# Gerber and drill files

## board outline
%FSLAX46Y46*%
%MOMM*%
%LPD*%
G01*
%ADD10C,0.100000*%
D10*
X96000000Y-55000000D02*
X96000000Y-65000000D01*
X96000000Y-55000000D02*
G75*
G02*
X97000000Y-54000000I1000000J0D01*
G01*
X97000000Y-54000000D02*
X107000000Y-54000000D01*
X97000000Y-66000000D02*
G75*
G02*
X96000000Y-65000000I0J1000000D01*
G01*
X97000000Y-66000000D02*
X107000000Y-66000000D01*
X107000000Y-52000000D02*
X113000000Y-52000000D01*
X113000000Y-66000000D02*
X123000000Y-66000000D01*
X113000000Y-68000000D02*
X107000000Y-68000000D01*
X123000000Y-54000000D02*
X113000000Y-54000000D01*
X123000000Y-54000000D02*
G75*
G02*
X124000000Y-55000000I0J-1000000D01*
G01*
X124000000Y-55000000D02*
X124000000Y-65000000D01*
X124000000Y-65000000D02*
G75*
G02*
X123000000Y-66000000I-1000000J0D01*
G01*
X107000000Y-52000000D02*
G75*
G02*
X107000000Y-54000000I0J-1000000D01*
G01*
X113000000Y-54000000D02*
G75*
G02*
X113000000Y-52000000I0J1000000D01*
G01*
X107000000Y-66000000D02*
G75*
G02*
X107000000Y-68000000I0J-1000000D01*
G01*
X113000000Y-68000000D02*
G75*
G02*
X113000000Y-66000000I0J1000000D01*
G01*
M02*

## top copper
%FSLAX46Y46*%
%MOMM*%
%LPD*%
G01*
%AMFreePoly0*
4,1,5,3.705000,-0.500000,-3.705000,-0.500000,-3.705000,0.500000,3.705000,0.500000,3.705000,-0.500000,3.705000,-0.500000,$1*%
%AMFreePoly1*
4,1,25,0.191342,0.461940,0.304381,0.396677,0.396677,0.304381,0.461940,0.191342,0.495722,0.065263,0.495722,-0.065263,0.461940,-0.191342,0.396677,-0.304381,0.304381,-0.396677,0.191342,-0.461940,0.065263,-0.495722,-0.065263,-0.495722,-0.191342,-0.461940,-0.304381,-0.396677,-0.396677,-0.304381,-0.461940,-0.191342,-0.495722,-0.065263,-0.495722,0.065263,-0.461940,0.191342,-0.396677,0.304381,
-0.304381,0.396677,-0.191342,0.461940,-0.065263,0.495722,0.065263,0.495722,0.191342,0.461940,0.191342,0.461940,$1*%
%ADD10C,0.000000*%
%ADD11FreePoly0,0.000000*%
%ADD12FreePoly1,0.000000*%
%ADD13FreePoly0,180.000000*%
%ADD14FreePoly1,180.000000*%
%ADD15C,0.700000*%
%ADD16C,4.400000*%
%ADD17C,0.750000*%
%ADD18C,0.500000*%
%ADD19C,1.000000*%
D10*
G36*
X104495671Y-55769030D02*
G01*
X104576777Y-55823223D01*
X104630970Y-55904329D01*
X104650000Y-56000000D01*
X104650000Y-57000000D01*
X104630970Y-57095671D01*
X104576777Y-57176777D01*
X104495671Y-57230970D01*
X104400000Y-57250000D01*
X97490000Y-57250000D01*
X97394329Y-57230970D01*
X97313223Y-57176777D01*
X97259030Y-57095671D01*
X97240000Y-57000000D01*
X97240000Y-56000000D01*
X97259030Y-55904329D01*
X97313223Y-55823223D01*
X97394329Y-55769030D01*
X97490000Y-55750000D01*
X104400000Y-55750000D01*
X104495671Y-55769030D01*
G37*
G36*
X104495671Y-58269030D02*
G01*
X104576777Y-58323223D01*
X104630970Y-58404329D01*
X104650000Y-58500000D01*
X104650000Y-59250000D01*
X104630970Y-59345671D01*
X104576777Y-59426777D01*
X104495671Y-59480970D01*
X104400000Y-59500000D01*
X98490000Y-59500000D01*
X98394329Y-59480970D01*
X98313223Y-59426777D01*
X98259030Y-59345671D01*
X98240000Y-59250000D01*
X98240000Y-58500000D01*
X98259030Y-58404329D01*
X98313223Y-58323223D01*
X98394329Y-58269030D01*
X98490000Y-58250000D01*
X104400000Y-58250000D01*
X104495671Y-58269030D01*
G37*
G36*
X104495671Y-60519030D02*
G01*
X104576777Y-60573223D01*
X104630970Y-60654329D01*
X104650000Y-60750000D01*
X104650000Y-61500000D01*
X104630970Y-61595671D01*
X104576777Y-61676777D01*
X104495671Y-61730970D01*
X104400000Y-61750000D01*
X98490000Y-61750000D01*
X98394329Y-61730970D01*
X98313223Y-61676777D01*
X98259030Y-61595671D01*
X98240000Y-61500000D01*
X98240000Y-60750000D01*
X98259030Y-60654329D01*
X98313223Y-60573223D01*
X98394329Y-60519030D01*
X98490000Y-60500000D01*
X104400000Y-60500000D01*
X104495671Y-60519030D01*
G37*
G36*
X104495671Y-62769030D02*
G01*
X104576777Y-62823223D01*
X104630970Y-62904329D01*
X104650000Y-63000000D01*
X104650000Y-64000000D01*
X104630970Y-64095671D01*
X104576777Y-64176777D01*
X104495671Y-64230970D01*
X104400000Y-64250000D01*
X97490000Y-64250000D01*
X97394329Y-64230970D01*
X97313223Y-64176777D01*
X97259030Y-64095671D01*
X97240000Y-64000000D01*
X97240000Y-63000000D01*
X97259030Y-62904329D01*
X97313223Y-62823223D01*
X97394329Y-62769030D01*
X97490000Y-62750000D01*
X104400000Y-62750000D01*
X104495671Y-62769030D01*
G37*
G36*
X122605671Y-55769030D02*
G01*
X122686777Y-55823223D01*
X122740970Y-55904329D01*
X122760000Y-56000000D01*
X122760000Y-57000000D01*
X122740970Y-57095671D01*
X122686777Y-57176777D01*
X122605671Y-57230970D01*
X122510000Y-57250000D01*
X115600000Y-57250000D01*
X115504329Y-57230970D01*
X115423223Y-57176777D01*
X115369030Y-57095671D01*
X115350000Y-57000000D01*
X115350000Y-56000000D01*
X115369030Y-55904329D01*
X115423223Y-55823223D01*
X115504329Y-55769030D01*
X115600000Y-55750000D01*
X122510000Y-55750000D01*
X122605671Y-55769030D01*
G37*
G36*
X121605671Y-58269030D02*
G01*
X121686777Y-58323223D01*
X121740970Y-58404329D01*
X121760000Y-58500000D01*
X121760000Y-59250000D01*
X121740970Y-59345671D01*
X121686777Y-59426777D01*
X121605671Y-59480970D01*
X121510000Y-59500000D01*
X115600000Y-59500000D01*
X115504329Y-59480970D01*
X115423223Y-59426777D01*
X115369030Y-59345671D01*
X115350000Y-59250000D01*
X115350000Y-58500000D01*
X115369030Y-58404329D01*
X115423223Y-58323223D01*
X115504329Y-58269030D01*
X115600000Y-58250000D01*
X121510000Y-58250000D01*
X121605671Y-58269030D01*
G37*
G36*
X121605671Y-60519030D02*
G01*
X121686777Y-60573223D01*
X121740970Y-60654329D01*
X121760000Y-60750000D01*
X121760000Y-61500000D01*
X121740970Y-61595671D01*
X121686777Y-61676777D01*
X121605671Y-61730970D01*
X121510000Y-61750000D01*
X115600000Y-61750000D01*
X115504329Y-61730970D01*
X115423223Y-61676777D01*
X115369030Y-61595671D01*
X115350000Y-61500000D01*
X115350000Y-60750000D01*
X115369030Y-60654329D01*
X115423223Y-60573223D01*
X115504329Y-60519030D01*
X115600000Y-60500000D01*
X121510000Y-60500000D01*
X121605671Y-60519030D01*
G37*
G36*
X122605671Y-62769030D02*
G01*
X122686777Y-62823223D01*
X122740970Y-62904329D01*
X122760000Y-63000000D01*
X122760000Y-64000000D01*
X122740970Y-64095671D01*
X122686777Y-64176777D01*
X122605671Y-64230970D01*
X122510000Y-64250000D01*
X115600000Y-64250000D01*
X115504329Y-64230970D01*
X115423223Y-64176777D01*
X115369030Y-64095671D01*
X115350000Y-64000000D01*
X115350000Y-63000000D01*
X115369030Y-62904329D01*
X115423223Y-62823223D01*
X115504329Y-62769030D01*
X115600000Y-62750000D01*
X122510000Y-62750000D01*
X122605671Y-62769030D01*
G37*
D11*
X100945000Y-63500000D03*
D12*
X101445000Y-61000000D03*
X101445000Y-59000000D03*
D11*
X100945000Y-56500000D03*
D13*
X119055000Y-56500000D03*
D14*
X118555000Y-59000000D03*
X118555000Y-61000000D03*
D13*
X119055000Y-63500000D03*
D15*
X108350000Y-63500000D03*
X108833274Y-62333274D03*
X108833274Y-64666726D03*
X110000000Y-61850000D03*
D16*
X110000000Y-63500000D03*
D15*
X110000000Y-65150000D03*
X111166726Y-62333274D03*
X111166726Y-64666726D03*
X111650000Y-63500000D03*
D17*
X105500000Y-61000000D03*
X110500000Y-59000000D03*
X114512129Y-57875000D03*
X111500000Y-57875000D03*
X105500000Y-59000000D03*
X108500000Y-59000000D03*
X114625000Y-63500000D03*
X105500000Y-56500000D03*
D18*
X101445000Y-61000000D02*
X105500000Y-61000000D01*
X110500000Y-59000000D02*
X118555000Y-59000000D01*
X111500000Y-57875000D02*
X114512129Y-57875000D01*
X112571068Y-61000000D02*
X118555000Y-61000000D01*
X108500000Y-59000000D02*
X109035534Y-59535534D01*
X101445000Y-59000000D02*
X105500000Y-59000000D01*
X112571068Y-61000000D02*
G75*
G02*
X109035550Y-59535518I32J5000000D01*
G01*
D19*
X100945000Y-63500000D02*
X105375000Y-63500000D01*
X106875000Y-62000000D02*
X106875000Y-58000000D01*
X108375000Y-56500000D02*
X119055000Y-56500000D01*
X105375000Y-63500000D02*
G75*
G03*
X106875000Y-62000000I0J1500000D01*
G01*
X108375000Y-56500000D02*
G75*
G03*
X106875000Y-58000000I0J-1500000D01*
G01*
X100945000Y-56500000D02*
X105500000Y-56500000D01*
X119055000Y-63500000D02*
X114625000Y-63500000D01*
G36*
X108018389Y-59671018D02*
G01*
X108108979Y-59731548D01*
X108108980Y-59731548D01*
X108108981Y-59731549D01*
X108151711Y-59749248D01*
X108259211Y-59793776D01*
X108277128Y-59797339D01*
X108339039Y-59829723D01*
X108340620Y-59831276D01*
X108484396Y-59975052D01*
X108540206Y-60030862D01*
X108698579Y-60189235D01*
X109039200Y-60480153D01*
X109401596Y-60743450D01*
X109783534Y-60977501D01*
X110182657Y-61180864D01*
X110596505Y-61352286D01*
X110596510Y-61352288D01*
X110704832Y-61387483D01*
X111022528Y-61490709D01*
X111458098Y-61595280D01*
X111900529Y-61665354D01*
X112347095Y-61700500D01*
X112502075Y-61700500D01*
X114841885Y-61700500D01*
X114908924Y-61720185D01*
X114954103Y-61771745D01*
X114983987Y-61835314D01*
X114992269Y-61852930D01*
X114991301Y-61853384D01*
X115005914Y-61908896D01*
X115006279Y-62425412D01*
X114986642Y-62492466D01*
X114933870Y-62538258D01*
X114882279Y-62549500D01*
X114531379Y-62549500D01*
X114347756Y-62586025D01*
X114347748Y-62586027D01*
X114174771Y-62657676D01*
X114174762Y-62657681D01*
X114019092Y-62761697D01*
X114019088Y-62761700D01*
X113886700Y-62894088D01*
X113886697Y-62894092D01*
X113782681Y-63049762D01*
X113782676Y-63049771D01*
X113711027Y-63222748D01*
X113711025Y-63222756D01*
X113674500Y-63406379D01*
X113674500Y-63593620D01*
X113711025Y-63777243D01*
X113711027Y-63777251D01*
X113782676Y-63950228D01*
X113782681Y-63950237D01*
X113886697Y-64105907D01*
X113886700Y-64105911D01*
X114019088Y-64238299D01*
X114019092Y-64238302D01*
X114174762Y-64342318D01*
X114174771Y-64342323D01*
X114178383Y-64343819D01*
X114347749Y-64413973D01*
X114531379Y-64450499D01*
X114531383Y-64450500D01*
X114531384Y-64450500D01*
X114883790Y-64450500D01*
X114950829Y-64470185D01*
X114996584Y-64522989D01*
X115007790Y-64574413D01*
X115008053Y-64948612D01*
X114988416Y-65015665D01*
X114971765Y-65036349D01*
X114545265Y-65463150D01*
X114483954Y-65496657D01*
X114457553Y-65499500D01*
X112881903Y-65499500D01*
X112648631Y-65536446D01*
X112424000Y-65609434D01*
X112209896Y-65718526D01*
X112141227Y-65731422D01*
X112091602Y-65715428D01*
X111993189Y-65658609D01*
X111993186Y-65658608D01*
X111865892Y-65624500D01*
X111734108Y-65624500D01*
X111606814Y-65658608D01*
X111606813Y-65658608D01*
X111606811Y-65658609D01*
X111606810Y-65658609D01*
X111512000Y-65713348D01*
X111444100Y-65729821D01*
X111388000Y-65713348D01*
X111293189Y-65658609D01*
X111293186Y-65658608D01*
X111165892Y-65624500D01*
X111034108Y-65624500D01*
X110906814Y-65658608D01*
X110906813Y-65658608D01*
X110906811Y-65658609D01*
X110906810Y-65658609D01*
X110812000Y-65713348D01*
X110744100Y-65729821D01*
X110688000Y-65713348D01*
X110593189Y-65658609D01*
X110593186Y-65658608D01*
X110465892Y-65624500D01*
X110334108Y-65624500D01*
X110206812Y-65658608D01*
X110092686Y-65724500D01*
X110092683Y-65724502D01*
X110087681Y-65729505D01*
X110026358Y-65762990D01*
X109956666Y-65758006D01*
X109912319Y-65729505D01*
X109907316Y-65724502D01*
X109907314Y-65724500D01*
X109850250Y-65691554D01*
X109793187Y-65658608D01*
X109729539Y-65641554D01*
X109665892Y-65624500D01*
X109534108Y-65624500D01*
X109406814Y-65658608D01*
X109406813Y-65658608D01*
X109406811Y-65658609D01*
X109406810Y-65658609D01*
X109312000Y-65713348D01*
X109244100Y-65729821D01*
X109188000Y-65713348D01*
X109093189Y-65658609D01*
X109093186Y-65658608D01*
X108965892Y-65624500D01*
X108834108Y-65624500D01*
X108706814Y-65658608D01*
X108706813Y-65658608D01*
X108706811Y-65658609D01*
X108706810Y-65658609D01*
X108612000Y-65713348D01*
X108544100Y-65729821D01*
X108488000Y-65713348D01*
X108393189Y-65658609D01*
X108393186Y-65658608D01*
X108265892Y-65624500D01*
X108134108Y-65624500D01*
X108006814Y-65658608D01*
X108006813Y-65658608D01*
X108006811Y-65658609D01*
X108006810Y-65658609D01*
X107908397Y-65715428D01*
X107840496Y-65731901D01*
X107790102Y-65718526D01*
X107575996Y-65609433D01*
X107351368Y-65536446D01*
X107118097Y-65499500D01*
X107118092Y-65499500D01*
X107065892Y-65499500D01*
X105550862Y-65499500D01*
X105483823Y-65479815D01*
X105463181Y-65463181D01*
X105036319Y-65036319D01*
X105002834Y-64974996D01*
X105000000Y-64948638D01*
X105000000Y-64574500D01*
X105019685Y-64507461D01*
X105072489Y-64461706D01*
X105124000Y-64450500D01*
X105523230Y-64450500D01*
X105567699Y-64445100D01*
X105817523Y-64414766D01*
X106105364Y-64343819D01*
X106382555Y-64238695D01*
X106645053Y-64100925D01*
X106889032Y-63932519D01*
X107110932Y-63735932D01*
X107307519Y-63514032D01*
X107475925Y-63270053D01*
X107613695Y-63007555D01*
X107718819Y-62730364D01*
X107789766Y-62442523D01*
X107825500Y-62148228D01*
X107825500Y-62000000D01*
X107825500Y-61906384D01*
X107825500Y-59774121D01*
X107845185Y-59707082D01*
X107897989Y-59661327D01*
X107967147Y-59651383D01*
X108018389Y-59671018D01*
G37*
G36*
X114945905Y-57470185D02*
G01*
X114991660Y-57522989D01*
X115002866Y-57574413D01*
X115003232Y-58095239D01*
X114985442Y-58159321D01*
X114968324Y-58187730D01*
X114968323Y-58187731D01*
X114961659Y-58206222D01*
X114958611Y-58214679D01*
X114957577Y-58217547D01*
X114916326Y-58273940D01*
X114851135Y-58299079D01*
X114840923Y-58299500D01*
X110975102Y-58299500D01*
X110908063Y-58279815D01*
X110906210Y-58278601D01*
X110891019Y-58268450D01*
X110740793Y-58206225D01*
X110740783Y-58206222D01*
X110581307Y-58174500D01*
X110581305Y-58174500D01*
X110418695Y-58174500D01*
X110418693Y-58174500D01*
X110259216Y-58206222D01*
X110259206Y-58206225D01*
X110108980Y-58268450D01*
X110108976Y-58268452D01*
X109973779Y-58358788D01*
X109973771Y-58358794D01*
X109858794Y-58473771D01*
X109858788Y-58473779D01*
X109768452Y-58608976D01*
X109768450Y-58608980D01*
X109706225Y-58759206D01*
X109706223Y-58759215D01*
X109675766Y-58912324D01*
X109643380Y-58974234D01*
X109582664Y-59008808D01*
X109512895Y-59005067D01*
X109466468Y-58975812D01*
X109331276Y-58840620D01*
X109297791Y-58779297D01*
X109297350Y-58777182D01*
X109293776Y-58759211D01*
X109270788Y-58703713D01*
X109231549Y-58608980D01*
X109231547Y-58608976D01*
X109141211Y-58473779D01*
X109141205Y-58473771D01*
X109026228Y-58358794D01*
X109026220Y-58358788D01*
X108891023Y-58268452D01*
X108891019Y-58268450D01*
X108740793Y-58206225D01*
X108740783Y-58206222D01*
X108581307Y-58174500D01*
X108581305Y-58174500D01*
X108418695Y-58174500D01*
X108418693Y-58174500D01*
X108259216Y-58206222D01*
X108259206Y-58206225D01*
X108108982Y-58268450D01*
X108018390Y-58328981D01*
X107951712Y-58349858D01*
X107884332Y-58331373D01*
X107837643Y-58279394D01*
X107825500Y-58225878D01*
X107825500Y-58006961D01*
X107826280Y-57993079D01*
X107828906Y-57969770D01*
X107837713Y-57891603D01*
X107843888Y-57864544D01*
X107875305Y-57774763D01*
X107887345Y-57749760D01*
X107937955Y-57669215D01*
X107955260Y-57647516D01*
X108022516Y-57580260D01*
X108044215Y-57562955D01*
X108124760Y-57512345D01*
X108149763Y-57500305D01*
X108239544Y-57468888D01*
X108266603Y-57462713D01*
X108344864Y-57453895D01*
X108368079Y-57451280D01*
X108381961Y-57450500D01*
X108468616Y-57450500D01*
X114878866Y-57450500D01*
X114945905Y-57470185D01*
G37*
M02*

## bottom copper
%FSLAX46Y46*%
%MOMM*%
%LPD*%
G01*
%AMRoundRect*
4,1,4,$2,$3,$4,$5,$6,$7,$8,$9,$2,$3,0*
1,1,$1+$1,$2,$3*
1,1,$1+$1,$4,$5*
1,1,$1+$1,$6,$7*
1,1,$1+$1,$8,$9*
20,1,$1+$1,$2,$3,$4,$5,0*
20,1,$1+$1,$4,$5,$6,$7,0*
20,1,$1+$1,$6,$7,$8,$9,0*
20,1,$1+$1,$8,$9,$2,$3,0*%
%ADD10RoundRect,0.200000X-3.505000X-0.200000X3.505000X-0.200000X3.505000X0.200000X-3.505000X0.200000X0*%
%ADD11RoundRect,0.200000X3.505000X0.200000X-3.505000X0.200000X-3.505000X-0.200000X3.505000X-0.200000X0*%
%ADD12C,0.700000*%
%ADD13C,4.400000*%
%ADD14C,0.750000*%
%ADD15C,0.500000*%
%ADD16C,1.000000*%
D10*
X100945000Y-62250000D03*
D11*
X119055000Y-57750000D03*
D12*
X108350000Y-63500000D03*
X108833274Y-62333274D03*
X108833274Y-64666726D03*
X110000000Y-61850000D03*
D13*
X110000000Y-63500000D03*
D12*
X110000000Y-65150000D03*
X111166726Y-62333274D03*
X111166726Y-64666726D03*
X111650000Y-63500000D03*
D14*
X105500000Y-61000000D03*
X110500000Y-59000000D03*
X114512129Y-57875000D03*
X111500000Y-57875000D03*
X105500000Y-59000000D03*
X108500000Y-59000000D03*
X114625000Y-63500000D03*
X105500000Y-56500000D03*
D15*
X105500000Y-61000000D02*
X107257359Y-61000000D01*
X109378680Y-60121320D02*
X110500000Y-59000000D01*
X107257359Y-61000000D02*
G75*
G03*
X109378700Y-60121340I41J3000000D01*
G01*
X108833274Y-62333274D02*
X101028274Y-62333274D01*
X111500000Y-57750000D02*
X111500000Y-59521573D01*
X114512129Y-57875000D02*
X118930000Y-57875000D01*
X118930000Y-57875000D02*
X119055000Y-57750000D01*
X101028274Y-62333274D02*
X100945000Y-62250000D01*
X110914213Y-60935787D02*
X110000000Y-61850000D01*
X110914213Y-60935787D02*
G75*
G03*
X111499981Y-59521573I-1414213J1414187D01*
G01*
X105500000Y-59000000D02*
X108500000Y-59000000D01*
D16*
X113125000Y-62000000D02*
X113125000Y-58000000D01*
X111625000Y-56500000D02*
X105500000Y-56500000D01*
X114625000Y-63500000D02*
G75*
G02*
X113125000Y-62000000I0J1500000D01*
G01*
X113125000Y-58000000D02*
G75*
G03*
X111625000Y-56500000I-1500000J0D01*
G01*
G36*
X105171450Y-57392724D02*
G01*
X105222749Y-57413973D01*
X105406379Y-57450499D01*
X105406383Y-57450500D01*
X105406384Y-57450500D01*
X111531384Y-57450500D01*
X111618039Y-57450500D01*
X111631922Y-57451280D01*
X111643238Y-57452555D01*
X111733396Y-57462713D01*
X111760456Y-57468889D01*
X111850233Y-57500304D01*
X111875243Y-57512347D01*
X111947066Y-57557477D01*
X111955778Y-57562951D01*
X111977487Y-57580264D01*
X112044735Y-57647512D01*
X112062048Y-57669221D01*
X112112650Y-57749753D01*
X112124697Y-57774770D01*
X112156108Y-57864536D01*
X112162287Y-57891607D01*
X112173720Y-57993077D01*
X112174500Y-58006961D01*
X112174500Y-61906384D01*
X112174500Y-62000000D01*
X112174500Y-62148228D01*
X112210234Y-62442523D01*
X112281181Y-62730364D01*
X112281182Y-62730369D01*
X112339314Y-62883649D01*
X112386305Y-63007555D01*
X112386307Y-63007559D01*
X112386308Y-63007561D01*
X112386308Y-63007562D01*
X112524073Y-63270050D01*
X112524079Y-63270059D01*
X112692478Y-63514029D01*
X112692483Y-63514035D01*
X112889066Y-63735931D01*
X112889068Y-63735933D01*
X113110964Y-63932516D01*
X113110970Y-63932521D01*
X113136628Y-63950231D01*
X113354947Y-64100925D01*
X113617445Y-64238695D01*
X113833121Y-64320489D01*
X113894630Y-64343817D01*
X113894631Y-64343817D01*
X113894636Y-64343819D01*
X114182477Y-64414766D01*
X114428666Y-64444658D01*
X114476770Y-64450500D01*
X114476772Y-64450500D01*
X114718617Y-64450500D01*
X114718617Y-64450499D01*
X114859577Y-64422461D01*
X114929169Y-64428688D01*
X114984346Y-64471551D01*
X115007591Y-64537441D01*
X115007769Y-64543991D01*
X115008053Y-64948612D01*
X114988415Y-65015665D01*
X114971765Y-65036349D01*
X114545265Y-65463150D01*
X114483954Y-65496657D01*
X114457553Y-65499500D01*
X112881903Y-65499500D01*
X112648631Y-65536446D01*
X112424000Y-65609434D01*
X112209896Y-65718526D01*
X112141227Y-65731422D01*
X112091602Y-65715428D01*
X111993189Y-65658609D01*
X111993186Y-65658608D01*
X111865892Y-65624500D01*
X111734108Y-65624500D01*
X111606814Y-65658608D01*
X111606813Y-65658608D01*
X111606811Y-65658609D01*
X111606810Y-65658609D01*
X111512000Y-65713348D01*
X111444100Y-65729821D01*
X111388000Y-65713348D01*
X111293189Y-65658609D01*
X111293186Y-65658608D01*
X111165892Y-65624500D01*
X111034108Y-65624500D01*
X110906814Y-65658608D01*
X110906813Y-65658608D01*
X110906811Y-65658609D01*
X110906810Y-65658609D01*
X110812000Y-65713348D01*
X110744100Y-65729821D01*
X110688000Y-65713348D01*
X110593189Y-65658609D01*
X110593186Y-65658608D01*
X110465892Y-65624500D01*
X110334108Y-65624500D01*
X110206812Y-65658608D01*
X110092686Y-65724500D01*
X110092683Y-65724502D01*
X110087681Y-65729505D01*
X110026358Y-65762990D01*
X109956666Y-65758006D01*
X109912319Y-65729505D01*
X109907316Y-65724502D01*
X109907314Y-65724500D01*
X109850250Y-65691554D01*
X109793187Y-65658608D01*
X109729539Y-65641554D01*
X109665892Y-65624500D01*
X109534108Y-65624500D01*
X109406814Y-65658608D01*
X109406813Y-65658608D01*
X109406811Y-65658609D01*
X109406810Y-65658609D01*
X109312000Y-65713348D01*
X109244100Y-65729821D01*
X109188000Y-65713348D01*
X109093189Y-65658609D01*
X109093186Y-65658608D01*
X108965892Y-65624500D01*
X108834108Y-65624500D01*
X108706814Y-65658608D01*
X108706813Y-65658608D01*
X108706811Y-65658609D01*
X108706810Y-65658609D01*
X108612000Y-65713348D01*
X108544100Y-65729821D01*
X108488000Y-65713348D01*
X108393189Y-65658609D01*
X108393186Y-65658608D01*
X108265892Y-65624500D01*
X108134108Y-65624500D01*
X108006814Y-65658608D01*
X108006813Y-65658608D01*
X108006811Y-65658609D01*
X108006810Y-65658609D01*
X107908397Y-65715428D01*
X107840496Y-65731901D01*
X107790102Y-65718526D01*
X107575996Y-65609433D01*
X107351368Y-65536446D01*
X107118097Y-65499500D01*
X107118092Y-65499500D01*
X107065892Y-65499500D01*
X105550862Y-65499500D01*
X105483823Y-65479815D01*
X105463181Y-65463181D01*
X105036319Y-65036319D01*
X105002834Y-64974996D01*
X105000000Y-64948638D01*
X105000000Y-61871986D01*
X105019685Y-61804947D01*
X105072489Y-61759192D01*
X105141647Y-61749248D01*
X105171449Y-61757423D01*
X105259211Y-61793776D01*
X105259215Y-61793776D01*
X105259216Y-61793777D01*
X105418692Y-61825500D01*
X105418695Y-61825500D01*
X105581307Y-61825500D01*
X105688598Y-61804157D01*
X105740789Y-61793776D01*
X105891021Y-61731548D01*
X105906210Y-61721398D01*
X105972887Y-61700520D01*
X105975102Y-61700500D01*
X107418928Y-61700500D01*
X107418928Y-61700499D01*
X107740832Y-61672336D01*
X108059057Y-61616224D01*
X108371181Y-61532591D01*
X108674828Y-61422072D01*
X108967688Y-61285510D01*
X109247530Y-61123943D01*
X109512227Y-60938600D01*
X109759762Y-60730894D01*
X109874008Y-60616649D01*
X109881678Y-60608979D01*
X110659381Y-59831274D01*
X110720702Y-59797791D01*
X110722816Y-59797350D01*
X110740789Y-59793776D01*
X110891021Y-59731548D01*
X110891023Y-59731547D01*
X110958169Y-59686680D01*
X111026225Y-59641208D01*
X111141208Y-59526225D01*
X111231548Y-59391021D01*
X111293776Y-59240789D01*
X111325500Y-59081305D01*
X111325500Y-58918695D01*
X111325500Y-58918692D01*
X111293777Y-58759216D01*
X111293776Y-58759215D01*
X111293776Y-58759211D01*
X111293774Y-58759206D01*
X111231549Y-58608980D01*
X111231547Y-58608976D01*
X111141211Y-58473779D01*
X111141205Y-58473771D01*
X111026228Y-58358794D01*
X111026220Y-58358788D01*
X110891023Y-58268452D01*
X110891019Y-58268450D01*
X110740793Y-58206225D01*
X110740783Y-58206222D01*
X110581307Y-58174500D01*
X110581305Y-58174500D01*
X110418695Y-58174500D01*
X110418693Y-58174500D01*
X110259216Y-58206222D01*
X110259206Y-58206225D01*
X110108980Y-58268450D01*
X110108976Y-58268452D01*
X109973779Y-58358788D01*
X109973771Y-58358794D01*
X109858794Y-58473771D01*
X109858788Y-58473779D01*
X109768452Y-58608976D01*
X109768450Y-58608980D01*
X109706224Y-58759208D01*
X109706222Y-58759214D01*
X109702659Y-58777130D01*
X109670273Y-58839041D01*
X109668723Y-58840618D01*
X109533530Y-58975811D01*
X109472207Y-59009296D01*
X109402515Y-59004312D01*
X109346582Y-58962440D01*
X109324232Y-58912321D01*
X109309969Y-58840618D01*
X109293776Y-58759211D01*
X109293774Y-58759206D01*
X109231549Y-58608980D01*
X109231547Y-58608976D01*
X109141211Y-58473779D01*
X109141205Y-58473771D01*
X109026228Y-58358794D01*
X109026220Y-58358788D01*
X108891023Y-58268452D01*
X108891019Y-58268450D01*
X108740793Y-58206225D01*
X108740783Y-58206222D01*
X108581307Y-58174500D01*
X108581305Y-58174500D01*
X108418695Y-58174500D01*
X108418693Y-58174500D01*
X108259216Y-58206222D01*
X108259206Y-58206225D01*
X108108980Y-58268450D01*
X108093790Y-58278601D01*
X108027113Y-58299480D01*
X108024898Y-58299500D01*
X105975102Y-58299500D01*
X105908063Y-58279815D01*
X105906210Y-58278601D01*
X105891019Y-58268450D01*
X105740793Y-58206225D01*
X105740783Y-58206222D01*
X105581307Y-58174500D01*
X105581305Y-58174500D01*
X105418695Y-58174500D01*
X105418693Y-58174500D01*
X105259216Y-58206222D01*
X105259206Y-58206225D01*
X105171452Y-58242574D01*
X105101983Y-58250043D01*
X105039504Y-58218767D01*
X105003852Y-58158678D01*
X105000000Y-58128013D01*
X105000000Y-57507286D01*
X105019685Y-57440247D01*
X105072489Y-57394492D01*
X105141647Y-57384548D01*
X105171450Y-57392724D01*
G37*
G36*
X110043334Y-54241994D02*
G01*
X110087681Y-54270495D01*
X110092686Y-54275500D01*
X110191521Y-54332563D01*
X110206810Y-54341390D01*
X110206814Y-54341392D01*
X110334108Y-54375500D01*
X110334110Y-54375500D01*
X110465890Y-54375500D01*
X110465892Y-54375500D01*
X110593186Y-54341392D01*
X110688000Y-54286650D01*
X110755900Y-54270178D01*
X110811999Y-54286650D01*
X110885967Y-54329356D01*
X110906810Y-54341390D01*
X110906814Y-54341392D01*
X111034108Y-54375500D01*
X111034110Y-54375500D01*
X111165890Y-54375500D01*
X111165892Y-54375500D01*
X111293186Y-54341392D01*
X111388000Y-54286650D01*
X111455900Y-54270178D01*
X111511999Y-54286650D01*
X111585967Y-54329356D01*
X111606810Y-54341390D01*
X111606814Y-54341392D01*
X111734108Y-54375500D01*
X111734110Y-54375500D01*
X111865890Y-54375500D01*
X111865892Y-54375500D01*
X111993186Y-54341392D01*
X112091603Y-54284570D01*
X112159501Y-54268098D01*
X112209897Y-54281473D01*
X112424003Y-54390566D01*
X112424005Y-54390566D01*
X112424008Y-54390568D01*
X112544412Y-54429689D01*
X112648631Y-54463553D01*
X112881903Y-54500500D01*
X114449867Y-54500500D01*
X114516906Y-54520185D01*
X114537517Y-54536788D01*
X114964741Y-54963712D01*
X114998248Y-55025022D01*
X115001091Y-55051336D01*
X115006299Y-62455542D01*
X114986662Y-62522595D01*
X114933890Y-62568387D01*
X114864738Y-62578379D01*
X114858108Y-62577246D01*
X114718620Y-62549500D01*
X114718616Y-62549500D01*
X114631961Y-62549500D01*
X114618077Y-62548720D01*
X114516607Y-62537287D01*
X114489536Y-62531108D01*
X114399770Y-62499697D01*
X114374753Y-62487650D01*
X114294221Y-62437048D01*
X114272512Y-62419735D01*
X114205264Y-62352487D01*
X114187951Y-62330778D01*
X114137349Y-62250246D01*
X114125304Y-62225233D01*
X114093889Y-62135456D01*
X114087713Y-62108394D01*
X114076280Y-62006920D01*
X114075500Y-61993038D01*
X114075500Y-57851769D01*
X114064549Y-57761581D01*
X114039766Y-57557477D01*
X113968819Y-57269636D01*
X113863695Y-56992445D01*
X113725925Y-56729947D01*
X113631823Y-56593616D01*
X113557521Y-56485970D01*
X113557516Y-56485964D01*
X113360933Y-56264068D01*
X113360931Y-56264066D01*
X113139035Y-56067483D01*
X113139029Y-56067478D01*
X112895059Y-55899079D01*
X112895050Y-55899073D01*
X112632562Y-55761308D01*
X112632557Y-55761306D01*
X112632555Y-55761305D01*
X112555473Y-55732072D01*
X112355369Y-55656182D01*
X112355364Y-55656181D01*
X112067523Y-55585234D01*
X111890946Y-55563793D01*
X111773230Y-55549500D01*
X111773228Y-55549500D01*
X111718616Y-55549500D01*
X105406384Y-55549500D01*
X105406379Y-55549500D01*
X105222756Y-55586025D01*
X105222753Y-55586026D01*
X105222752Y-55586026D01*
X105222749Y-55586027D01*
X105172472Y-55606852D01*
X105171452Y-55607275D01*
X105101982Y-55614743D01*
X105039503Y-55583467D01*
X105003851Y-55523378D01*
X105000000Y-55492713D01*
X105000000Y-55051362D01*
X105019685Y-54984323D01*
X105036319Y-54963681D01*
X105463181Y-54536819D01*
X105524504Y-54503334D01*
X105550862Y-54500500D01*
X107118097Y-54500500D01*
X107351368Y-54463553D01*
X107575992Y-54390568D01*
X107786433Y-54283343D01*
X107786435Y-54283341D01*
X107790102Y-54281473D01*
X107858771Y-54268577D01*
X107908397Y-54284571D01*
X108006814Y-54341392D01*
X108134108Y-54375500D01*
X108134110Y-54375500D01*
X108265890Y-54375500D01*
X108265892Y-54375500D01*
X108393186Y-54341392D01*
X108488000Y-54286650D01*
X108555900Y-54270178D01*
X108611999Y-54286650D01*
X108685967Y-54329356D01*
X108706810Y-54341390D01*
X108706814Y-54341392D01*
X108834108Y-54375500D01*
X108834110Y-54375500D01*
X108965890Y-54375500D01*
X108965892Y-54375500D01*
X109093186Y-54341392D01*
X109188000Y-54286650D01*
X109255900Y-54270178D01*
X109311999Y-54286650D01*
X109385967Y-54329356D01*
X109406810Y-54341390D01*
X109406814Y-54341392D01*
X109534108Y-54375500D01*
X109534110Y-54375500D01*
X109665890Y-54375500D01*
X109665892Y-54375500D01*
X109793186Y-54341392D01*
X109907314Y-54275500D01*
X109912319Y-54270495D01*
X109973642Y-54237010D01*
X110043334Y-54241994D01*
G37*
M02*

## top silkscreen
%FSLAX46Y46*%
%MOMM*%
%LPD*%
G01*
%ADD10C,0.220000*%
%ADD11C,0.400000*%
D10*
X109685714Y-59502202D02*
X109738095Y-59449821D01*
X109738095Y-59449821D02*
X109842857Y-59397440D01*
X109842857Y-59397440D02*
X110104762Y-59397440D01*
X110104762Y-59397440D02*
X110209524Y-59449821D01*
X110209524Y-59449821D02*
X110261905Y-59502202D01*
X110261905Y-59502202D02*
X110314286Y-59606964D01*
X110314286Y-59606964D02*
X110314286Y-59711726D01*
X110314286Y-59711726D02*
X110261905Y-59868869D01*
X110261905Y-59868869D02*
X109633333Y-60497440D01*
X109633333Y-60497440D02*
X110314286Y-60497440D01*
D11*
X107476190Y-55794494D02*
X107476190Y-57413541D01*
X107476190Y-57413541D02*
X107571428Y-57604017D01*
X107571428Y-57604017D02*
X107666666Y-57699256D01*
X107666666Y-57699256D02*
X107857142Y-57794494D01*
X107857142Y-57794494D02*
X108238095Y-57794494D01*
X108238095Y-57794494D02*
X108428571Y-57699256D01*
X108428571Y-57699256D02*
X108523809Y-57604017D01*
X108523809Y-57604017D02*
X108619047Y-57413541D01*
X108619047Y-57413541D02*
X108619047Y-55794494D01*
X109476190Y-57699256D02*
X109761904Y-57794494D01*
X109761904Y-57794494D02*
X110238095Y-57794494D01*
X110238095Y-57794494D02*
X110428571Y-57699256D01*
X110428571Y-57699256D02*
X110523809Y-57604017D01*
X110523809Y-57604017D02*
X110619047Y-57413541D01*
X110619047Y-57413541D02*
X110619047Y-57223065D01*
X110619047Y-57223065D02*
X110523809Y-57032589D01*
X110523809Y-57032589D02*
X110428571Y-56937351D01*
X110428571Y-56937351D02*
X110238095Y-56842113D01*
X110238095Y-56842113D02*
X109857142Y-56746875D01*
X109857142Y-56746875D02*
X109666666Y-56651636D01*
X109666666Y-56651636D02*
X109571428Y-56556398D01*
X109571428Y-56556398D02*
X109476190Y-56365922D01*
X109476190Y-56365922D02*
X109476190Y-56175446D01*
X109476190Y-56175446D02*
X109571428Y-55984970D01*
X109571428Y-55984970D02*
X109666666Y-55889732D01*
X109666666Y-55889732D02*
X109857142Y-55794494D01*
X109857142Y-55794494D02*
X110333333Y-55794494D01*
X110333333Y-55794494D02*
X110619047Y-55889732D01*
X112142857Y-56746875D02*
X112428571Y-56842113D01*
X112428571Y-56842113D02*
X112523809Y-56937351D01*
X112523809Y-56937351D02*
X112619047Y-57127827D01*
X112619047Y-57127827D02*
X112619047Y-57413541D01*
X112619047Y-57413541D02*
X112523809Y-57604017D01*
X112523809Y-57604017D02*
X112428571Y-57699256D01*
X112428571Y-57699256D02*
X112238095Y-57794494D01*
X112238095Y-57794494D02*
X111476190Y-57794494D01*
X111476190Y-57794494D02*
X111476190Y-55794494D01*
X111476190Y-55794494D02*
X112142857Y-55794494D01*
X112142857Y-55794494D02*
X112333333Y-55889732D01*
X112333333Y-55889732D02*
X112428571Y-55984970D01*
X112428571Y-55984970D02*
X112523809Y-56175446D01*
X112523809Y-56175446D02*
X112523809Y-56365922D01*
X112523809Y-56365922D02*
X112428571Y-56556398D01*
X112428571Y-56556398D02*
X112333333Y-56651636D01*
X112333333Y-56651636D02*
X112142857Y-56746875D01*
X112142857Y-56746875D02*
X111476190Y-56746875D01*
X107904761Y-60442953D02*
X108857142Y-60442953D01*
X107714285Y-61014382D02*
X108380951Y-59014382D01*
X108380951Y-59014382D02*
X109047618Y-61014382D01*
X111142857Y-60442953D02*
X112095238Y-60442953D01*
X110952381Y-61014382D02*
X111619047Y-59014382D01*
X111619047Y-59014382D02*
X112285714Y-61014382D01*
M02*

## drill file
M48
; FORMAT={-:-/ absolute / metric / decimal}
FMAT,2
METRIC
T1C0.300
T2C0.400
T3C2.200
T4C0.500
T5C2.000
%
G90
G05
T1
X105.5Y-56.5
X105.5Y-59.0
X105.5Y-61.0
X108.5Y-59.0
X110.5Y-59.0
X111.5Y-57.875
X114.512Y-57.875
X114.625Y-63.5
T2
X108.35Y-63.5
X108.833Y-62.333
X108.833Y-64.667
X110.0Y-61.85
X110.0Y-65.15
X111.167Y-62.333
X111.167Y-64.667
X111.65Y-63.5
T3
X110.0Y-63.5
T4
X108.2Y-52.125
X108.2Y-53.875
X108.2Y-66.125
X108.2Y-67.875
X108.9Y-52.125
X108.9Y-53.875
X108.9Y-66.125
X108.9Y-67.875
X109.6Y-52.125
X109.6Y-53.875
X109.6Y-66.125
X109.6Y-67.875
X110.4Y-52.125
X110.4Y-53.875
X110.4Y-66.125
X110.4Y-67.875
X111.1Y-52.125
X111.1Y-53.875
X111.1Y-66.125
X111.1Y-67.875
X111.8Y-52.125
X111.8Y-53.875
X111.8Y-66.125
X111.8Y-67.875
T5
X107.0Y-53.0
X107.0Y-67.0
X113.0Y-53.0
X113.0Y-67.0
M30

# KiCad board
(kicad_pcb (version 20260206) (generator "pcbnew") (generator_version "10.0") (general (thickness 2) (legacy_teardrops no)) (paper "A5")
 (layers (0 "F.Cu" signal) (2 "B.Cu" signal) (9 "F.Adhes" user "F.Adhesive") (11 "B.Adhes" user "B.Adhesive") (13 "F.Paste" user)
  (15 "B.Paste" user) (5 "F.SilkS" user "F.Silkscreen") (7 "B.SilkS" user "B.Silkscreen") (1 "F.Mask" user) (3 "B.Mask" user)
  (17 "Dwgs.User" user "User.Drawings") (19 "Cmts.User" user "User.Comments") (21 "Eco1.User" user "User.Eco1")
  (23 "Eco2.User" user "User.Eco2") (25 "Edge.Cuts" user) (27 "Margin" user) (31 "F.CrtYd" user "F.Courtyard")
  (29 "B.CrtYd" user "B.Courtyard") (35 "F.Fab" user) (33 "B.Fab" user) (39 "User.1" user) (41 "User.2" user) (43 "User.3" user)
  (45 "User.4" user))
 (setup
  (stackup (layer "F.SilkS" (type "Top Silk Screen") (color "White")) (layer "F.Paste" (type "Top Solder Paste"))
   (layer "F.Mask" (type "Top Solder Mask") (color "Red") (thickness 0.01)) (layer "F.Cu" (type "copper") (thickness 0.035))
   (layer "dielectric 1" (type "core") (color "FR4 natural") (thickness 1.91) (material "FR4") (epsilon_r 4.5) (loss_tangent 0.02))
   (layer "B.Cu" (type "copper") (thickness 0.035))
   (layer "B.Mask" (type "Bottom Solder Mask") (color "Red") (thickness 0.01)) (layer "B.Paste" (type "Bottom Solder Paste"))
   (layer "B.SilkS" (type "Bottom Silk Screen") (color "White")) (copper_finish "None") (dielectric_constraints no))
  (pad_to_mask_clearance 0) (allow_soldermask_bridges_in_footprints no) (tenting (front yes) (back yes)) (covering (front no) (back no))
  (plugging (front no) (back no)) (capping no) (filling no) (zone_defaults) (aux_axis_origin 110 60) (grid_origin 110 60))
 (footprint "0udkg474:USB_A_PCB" (layer "F.Cu") (at 104.88 60)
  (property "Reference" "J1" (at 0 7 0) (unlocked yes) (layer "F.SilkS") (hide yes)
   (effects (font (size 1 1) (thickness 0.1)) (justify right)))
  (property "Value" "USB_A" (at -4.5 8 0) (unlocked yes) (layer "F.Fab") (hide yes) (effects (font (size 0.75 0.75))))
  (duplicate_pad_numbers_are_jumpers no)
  (fp_poly
   (pts (xy -0.384329 -4.23097) (xy -0.303223 -4.176777) (xy -0.24903 -4.095671) (xy -0.23 -4) (xy -0.23 -3) (xy -0.24903 -2.904329)
    (xy -0.303223 -2.823223) (xy -0.384329 -2.76903) (xy -0.48 -2.75) (xy -7.39 -2.75) (xy -7.485671 -2.76903) (xy -7.566777 -2.823223)
    (xy -7.62097 -2.904329) (xy -7.64 -3) (xy -7.64 -4) (xy -7.62097 -4.095671) (xy -7.566777 -4.176777) (xy -7.485671 -4.23097)
    (xy -7.39 -4.25) (xy -0.48 -4.25))
   (stroke (width 0) (type solid)) (fill yes) (layer "F.Cu"))
  (fp_poly
   (pts (xy -0.384329 -1.73097) (xy -0.303223 -1.676777) (xy -0.24903 -1.595671) (xy -0.23 -1.5) (xy -0.23 -0.75) (xy -0.24903 -0.654329)
    (xy -0.303223 -0.573223) (xy -0.384329 -0.51903) (xy -0.48 -0.5) (xy -6.39 -0.5) (xy -6.485671 -0.51903) (xy -6.566777 -0.573223)
    (xy -6.62097 -0.654329) (xy -6.64 -0.75) (xy -6.64 -1.5) (xy -6.62097 -1.595671) (xy -6.566777 -1.676777) (xy -6.485671 -1.73097)
    (xy -6.39 -1.75) (xy -0.48 -1.75))
   (stroke (width 0) (type solid)) (fill yes) (layer "F.Cu"))
  (fp_poly
   (pts (xy -0.384329 0.51903) (xy -0.303223 0.573223) (xy -0.24903 0.654329) (xy -0.23 0.75) (xy -0.23 1.5) (xy -0.24903 1.595671)
    (xy -0.303223 1.676777) (xy -0.384329 1.73097) (xy -0.48 1.75) (xy -6.39 1.75) (xy -6.485671 1.73097) (xy -6.566777 1.676777)
    (xy -6.62097 1.595671) (xy -6.64 1.5) (xy -6.64 0.75) (xy -6.62097 0.654329) (xy -6.566777 0.573223) (xy -6.485671 0.51903)
    (xy -6.39 0.5) (xy -0.48 0.5))
   (stroke (width 0) (type solid)) (fill yes) (layer "F.Cu"))
  (fp_poly
   (pts (xy -0.384329 2.76903) (xy -0.303223 2.823223) (xy -0.24903 2.904329) (xy -0.23 3) (xy -0.23 4) (xy -0.24903 4.095671)
    (xy -0.303223 4.176777) (xy -0.384329 4.23097) (xy -0.48 4.25) (xy -7.39 4.25) (xy -7.485671 4.23097) (xy -7.566777 4.176777)
    (xy -7.62097 4.095671) (xy -7.64 4) (xy -7.64 3) (xy -7.62097 2.904329) (xy -7.566777 2.823223) (xy -7.485671 2.76903) (xy -7.39 2.75)
    (xy -0.48 2.75))
   (stroke (width 0) (type solid)) (fill yes) (layer "F.Cu"))
  (pad "1" smd custom (at -3.935 3.5) (size 7.41 1) (layers "F.Cu" "F.Mask") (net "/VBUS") (solder_paste_margin 0)
   (options (clearance outline) (anchor rect)) (primitives))
  (pad "2" smd custom (at -3.435 1) (size 1 1) (layers "F.Cu" "F.Mask") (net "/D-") (solder_paste_margin 0) (thermal_bridge_angle 90)
   (options (clearance outline) (anchor circle)) (primitives))
  (pad "3" smd custom (at -3.435 -1) (size 1 1) (layers "F.Cu" "F.Mask") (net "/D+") (solder_paste_margin 0) (thermal_bridge_angle 90)
   (options (clearance outline) (anchor circle)) (primitives))
  (pad "4" smd custom (at -3.935 -3.5) (size 7.41 1) (layers "F.Cu" "F.Mask") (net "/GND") (solder_paste_margin 0)
   (options (clearance outline) (anchor rect)) (primitives))
  (pad "SH" smd roundrect (at -3.935 2.25) (size 7.41 0.8) (layers "B.Cu" "B.Mask") (roundrect_rratio 0.25) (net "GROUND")
   (solder_paste_margin 0))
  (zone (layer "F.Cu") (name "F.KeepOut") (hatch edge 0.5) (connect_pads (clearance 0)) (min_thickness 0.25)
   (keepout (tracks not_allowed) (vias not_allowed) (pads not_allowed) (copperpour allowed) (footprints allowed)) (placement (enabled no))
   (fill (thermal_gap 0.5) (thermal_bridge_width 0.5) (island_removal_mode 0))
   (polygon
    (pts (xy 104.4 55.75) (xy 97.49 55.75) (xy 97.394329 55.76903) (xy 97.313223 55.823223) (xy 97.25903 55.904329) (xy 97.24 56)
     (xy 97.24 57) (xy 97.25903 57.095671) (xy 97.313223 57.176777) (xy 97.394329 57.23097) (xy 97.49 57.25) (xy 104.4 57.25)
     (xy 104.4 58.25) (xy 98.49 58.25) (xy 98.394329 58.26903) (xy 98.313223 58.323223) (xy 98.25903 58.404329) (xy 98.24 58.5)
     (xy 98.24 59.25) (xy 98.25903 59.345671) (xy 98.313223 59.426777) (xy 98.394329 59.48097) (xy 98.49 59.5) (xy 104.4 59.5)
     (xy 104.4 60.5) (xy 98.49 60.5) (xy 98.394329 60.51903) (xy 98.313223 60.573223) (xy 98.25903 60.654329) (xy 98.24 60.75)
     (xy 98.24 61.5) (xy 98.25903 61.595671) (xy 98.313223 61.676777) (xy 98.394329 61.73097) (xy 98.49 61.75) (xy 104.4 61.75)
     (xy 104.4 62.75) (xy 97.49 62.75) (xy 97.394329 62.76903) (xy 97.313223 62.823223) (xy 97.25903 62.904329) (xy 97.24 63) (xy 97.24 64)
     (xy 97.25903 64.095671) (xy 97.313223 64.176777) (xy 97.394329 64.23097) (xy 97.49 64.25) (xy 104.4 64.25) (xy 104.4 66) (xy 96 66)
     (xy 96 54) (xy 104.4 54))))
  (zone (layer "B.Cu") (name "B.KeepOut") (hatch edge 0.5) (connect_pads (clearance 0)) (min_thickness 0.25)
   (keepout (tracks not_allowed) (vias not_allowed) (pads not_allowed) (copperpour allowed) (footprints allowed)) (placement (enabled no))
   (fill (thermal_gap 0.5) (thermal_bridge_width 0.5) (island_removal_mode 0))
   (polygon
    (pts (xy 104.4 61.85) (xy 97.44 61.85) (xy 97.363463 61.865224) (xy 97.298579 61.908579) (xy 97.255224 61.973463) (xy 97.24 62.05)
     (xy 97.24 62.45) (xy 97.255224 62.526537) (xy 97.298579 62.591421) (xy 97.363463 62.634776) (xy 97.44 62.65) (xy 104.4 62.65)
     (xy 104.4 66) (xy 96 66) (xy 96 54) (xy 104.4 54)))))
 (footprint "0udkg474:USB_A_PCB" (layer "F.Cu") (at 115.12 60 180)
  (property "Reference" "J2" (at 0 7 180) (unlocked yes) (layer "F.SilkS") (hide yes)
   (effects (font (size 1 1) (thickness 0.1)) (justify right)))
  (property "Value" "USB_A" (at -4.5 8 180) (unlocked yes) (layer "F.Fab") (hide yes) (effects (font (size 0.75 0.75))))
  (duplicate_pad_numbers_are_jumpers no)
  (fp_poly
   (pts (xy -0.384329 2.76903) (xy -0.303223 2.823223) (xy -0.24903 2.904329) (xy -0.23 3) (xy -0.23 4) (xy -0.24903 4.095671)
    (xy -0.303223 4.176777) (xy -0.384329 4.23097) (xy -0.48 4.25) (xy -7.39 4.25) (xy -7.485671 4.23097) (xy -7.566777 4.176777)
    (xy -7.62097 4.095671) (xy -7.64 4) (xy -7.64 3) (xy -7.62097 2.904329) (xy -7.566777 2.823223) (xy -7.485671 2.76903) (xy -7.39 2.75)
    (xy -0.48 2.75))
   (stroke (width 0) (type solid)) (fill yes) (layer "F.Cu"))
  (fp_poly
   (pts (xy -0.384329 0.51903) (xy -0.303223 0.573223) (xy -0.24903 0.654329) (xy -0.23 0.75) (xy -0.23 1.5) (xy -0.24903 1.595671)
    (xy -0.303223 1.676777) (xy -0.384329 1.73097) (xy -0.48 1.75) (xy -6.39 1.75) (xy -6.485671 1.73097) (xy -6.566777 1.676777)
    (xy -6.62097 1.595671) (xy -6.64 1.5) (xy -6.64 0.75) (xy -6.62097 0.654329) (xy -6.566777 0.573223) (xy -6.485671 0.51903)
    (xy -6.39 0.5) (xy -0.48 0.5))
   (stroke (width 0) (type solid)) (fill yes) (layer "F.Cu"))
  (fp_poly
   (pts (xy -0.384329 -1.73097) (xy -0.303223 -1.676777) (xy -0.24903 -1.595671) (xy -0.23 -1.5) (xy -0.23 -0.75) (xy -0.24903 -0.654329)
    (xy -0.303223 -0.573223) (xy -0.384329 -0.51903) (xy -0.48 -0.5) (xy -6.39 -0.5) (xy -6.485671 -0.51903) (xy -6.566777 -0.573223)
    (xy -6.62097 -0.654329) (xy -6.64 -0.75) (xy -6.64 -1.5) (xy -6.62097 -1.595671) (xy -6.566777 -1.676777) (xy -6.485671 -1.73097)
    (xy -6.39 -1.75) (xy -0.48 -1.75))
   (stroke (width 0) (type solid)) (fill yes) (layer "F.Cu"))
  (fp_poly
   (pts (xy -0.384329 -4.23097) (xy -0.303223 -4.176777) (xy -0.24903 -4.095671) (xy -0.23 -4) (xy -0.23 -3) (xy -0.24903 -2.904329)
    (xy -0.303223 -2.823223) (xy -0.384329 -2.76903) (xy -0.48 -2.75) (xy -7.39 -2.75) (xy -7.485671 -2.76903) (xy -7.566777 -2.823223)
    (xy -7.62097 -2.904329) (xy -7.64 -3) (xy -7.64 -4) (xy -7.62097 -4.095671) (xy -7.566777 -4.176777) (xy -7.485671 -4.23097)
    (xy -7.39 -4.25) (xy -0.48 -4.25))
   (stroke (width 0) (type solid)) (fill yes) (layer "F.Cu"))
  (pad "1" smd custom (at -3.935 3.5 180) (size 7.41 1) (layers "F.Cu" "F.Mask") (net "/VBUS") (solder_paste_margin 0)
   (options (clearance outline) (anchor rect)) (primitives))
  (pad "2" smd custom (at -3.435 1 180) (size 1 1) (layers "F.Cu" "F.Mask") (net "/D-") (solder_paste_margin 0) (thermal_bridge_angle 90)
   (options (clearance outline) (anchor circle)) (primitives))
  (pad "3" smd custom (at -3.435 -1 180) (size 1 1) (layers "F.Cu" "F.Mask") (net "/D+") (solder_paste_margin 0) (thermal_bridge_angle 90)
   (options (clearance outline) (anchor circle)) (primitives))
  (pad "4" smd custom (at -3.935 -3.5 180) (size 7.41 1) (layers "F.Cu" "F.Mask") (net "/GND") (solder_paste_margin 0)
   (options (clearance outline) (anchor rect)) (primitives))
  (pad "SH" smd roundrect (at -3.935 2.25 180) (size 7.41 0.8) (layers "B.Cu" "B.Mask") (roundrect_rratio 0.25) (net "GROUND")
   (solder_paste_margin 0))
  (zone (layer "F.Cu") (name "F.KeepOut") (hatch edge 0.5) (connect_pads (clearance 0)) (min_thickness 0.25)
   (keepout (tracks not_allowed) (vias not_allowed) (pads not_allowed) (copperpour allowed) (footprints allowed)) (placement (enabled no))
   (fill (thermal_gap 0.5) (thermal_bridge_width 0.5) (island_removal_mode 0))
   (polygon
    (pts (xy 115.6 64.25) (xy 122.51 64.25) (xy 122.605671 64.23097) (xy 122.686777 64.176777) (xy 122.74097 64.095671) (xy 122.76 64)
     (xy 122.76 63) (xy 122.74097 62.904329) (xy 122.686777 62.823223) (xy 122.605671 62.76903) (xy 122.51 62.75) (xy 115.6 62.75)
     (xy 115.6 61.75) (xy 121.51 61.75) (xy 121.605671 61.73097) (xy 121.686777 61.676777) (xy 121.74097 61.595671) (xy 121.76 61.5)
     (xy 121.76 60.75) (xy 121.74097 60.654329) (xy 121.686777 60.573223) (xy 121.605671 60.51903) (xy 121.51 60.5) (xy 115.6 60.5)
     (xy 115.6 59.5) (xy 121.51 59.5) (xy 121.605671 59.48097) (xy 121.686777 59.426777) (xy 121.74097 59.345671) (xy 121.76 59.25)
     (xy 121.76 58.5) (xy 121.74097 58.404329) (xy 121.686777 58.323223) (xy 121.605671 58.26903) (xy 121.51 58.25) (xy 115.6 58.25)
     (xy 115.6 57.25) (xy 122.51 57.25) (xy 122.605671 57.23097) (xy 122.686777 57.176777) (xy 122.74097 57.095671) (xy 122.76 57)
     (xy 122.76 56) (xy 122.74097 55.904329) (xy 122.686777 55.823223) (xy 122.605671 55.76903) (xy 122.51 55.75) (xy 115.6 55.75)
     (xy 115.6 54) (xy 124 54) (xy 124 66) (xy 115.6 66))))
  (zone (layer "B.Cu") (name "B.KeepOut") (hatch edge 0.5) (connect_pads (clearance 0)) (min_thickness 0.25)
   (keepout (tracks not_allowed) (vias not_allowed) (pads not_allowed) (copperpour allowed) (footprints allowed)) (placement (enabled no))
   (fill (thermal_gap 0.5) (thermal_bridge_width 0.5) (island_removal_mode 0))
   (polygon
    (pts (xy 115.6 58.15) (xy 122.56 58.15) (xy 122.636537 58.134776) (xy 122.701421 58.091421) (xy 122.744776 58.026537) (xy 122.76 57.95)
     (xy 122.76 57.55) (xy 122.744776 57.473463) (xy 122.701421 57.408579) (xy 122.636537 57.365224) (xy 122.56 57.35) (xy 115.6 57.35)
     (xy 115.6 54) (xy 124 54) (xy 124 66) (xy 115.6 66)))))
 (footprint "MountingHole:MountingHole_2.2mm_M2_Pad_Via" (layer "F.Cu") (at 110 63.5)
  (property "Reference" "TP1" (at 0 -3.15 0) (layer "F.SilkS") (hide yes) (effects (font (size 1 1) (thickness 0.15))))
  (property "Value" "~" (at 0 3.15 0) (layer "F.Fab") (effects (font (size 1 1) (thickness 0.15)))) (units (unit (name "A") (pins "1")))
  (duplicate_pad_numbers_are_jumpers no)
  (pad "1" thru_hole circle (at -1.65 0) (size 0.7 0.7) (drill 0.4) (layers "*.Cu" "*.Mask") (remove_unused_layers no) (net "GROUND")
   (zone_connect 2))
  (pad "1" thru_hole circle (at -1.166726 -1.166726) (size 0.7 0.7) (drill 0.4) (layers "*.Cu" "*.Mask") (remove_unused_layers no)
   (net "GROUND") (zone_connect 2))
  (pad "1" thru_hole circle (at -1.166726 1.166726) (size 0.7 0.7) (drill 0.4) (layers "*.Cu" "*.Mask") (remove_unused_layers no)
   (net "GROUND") (zone_connect 2))
  (pad "1" thru_hole circle (at 0 -1.65) (size 0.7 0.7) (drill 0.4) (layers "*.Cu" "*.Mask") (remove_unused_layers no) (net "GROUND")
   (zone_connect 2))
  (pad "1" thru_hole circle (at 0 0) (size 4.4 4.4) (drill 2.2) (layers "*.Cu" "*.Mask") (remove_unused_layers no) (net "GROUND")
   (zone_connect 2))
  (pad "1" thru_hole circle (at 0 1.65) (size 0.7 0.7) (drill 0.4) (layers "*.Cu" "*.Mask") (remove_unused_layers no) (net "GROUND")
   (zone_connect 2))
  (pad "1" thru_hole circle (at 1.166726 -1.166726) (size 0.7 0.7) (drill 0.4) (layers "*.Cu" "*.Mask") (remove_unused_layers no)
   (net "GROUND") (zone_connect 2))
  (pad "1" thru_hole circle (at 1.166726 1.166726) (size 0.7 0.7) (drill 0.4) (layers "*.Cu" "*.Mask") (remove_unused_layers no)
   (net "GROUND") (zone_connect 2))
  (pad "1" thru_hole circle (at 1.65 0) (size 0.7 0.7) (drill 0.4) (layers "*.Cu" "*.Mask") (remove_unused_layers no) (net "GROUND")
   (zone_connect 2)))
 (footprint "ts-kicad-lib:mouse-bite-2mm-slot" (layer "F.Cu") (at 110 53)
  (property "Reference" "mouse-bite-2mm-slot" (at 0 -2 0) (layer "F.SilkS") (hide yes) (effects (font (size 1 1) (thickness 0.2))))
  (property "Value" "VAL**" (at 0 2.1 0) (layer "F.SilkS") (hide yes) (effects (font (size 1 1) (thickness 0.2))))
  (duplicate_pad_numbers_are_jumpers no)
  (fp_arc (start -3 -1) (mid -2 0) (end -3 1) (stroke (width 0.1) (type solid)) (layer "Edge.Cuts"))
  (fp_arc (start 3 1) (mid 2 0) (end 3 -1) (stroke (width 0.1) (type solid)) (layer "Edge.Cuts"))
  (pad "" np_thru_hole circle (at -3 0) (size 0.5 0.5) (drill 2) (layers "*.Cu" "*.Mask"))
  (pad "" np_thru_hole circle (at -1.8 -0.875 180) (size 0.5 0.5) (drill 0.5) (layers "*.Cu" "*.Mask"))
  (pad "" np_thru_hole circle (at -1.8 0.875) (size 0.5 0.5) (drill 0.5) (layers "*.Cu" "*.Mask"))
  (pad "" np_thru_hole circle (at -1.1 -0.875 180) (size 0.5 0.5) (drill 0.5) (layers "*.Cu" "*.Mask"))
  (pad "" np_thru_hole circle (at -1.1 0.875) (size 0.5 0.5) (drill 0.5) (layers "*.Cu" "*.Mask"))
  (pad "" np_thru_hole circle (at -0.4 -0.875 180) (size 0.5 0.5) (drill 0.5) (layers "*.Cu" "*.Mask"))
  (pad "" np_thru_hole circle (at -0.4 0.875) (size 0.5 0.5) (drill 0.5) (layers "*.Cu" "*.Mask"))
  (pad "" np_thru_hole circle (at 0.4 -0.875 180) (size 0.5 0.5) (drill 0.5) (layers "*.Cu" "*.Mask"))
  (pad "" np_thru_hole circle (at 0.4 0.875) (size 0.5 0.5) (drill 0.5) (layers "*.Cu" "*.Mask"))
  (pad "" np_thru_hole circle (at 1.1 -0.875 180) (size 0.5 0.5) (drill 0.5) (layers "*.Cu" "*.Mask"))
  (pad "" np_thru_hole circle (at 1.1 0.875) (size 0.5 0.5) (drill 0.5) (layers "*.Cu" "*.Mask"))
  (pad "" np_thru_hole circle (at 1.8 -0.875 180) (size 0.5 0.5) (drill 0.5) (layers "*.Cu" "*.Mask"))
  (pad "" np_thru_hole circle (at 1.8 0.875) (size 0.5 0.5) (drill 0.5) (layers "*.Cu" "*.Mask"))
  (pad "" np_thru_hole circle (at 3 0) (size 0.5 0.5) (drill 2) (layers "*.Cu" "*.Mask")))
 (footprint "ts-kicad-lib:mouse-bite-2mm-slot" (layer "F.Cu") (at 110 67 180)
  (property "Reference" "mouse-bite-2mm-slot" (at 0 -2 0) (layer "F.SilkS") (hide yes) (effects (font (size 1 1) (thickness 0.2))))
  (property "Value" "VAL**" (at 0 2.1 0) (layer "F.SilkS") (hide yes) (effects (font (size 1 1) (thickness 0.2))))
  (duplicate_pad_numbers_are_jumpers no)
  (fp_arc (start 3 1) (mid 2 0) (end 3 -1) (stroke (width 0.1) (type solid)) (layer "Edge.Cuts"))
  (fp_arc (start -3 -1) (mid -2 0) (end -3 1) (stroke (width 0.1) (type solid)) (layer "Edge.Cuts"))
  (pad "" np_thru_hole circle (at -3 0 180) (size 0.5 0.5) (drill 2) (layers "*.Cu" "*.Mask"))
  (pad "" np_thru_hole circle (at -1.8 -0.875) (size 0.5 0.5) (drill 0.5) (layers "*.Cu" "*.Mask"))
  (pad "" np_thru_hole circle (at -1.8 0.875 180) (size 0.5 0.5) (drill 0.5) (layers "*.Cu" "*.Mask"))
  (pad "" np_thru_hole circle (at -1.1 -0.875) (size 0.5 0.5) (drill 0.5) (layers "*.Cu" "*.Mask"))
  (pad "" np_thru_hole circle (at -1.1 0.875 180) (size 0.5 0.5) (drill 0.5) (layers "*.Cu" "*.Mask"))
  (pad "" np_thru_hole circle (at -0.4 -0.875) (size 0.5 0.5) (drill 0.5) (layers "*.Cu" "*.Mask"))
  (pad "" np_thru_hole circle (at -0.4 0.875 180) (size 0.5 0.5) (drill 0.5) (layers "*.Cu" "*.Mask"))
  (pad "" np_thru_hole circle (at 0.4 -0.875) (size 0.5 0.5) (drill 0.5) (layers "*.Cu" "*.Mask"))
  (pad "" np_thru_hole circle (at 0.4 0.875 180) (size 0.5 0.5) (drill 0.5) (layers "*.Cu" "*.Mask"))
  (pad "" np_thru_hole circle (at 1.1 -0.875) (size 0.5 0.5) (drill 0.5) (layers "*.Cu" "*.Mask"))
  (pad "" np_thru_hole circle (at 1.1 0.875 180) (size 0.5 0.5) (drill 0.5) (layers "*.Cu" "*.Mask"))
  (pad "" np_thru_hole circle (at 1.8 -0.875) (size 0.5 0.5) (drill 0.5) (layers "*.Cu" "*.Mask"))
  (pad "" np_thru_hole circle (at 1.8 0.875 180) (size 0.5 0.5) (drill 0.5) (layers "*.Cu" "*.Mask"))
  (pad "" np_thru_hole circle (at 3 0 180) (size 0.5 0.5) (drill 2) (layers "*.Cu" "*.Mask")))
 (gr_line (start 96 55) (end 96 65) (stroke (width 0.1) (type solid)) (layer "Edge.Cuts"))
 (gr_arc (start 96 55) (mid 96.292893 54.292893) (end 97 54) (stroke (width 0.1) (type solid)) (layer "Edge.Cuts"))
 (gr_line (start 97 54) (end 107 54) (stroke (width 0.1) (type solid)) (layer "Edge.Cuts"))
 (gr_arc (start 97 66) (mid 96.292893 65.707107) (end 96 65) (stroke (width 0.1) (type solid)) (layer "Edge.Cuts"))
 (gr_line (start 97 66) (end 107 66) (stroke (width 0.1) (type solid)) (layer "Edge.Cuts"))
 (gr_line (start 107 52) (end 113 52) (stroke (width 0.1) (type solid)) (layer "Edge.Cuts"))
 (gr_line (start 113 66) (end 123 66) (stroke (width 0.1) (type solid)) (layer "Edge.Cuts"))
 (gr_line (start 113 68) (end 107 68) (stroke (width 0.1) (type solid)) (layer "Edge.Cuts"))
 (gr_line (start 123 54) (end 113 54) (stroke (width 0.1) (type solid)) (layer "Edge.Cuts"))
 (gr_arc (start 123 54) (mid 123.707107 54.292893) (end 124 55) (stroke (width 0.1) (type solid)) (layer "Edge.Cuts"))
 (gr_line (start 124 55) (end 124 65) (stroke (width 0.1) (type solid)) (layer "Edge.Cuts"))
 (gr_arc (start 124 65) (mid 123.707107 65.707107) (end 123 66) (stroke (width 0.1) (type solid)) (layer "Edge.Cuts"))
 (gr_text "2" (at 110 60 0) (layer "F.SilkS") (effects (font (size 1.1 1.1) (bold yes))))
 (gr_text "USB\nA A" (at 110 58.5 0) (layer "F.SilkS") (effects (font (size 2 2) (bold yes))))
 (segment (start 101.445 61) (end 105.5 61) (width 0.5) (layer "F.Cu") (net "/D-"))
 (segment (start 110.5 59) (end 118.555 59) (width 0.5) (layer "F.Cu") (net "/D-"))
 (via (at 105.5 61) (size 0.75) (drill 0.3) (layers "F.Cu" "B.Cu") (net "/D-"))
 (via (at 110.5 59) (size 0.75) (drill 0.3) (layers "F.Cu" "B.Cu") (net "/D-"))
 (segment (start 105.5 61) (end 107.257359 61) (width 0.5) (layer "B.Cu") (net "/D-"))
 (segment (start 109.37868 60.12132) (end 110.5 59) (width 0.5) (layer "B.Cu") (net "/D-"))
 (arc (start 107.257359 61) (mid 108.40541 60.771638) (end 109.37868 60.12132) (width 0.5) (layer "B.Cu") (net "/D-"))
 (segment (start 111.5 57.875) (end 114.512129 57.875) (width 0.5) (layer "F.Cu") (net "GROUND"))
 (via (at 114.512129 57.875) (size 0.75) (drill 0.3) (layers "F.Cu" "B.Cu") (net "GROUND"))
 (via (at 111.5 57.875) (size 0.75) (drill 0.3) (layers "F.Cu" "B.Cu") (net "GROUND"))
 (segment (start 108.833274 62.333274) (end 101.028274 62.333274) (width 0.5) (layer "B.Cu") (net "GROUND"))
 (segment (start 111.5 57.75) (end 111.5 59.521573) (width 0.5) (layer "B.Cu") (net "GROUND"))
 (segment (start 114.512129 57.875) (end 118.93 57.875) (width 0.5) (layer "B.Cu") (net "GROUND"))
 (segment (start 118.93 57.875) (end 119.055 57.75) (width 0.5) (layer "B.Cu") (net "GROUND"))
 (segment (start 101.028274 62.333274) (end 100.945 62.25) (width 0.5) (layer "B.Cu") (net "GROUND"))
 (segment (start 110.914213 60.935787) (end 110 61.85) (width 0.5) (layer "B.Cu") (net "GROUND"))
 (arc (start 110.914213 60.935787) (mid 111.347759 60.28694) (end 111.5 59.521573) (width 0.5) (layer "B.Cu") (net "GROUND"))
 (segment (start 112.571068 61) (end 118.555 61) (width 0.5) (layer "F.Cu") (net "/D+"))
 (segment (start 108.5 59) (end 109.035534 59.535534) (width 0.5) (layer "F.Cu") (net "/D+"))
 (segment (start 101.445 59) (end 105.5 59) (width 0.5) (layer "F.Cu") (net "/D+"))
 (via (at 105.5 59) (size 0.75) (drill 0.3) (layers "F.Cu" "B.Cu") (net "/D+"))
 (via (at 108.5 59) (size 0.75) (drill 0.3) (layers "F.Cu" "B.Cu") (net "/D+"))
 (arc (start 112.571068 61) (mid 110.657651 60.619398) (end 109.035534 59.535534) (width 0.5) (layer "F.Cu") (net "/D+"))
 (segment (start 105.5 59) (end 108.5 59) (width 0.5) (layer "B.Cu") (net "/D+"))
 (segment (start 100.945 63.5) (end 105.375 63.5) (width 1) (layer "F.Cu") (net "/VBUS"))
 (segment (start 106.875 62) (end 106.875 58) (width 1) (layer "F.Cu") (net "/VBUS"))
 (segment (start 108.375 56.5) (end 119.055 56.5) (width 1) (layer "F.Cu") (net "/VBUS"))
 (arc (start 105.375 63.5) (mid 106.43566 63.06066) (end 106.875 62) (width 1) (layer "F.Cu") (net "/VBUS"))
 (arc (start 108.375 56.5) (mid 107.31434 56.93934) (end 106.875 58) (width 1) (layer "F.Cu") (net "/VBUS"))
 (segment (start 100.945 56.5) (end 105.5 56.5) (width 1) (layer "F.Cu") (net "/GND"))
 (segment (start 119.055 63.5) (end 114.625 63.5) (width 1) (layer "F.Cu") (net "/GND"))
 (via (at 114.625 63.5) (size 0.75) (drill 0.3) (layers "F.Cu" "B.Cu") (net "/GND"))
 (via (at 105.5 56.5) (size 0.75) (drill 0.3) (layers "F.Cu" "B.Cu") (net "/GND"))
 (segment (start 113.125 62) (end 113.125 58) (width 1) (layer "B.Cu") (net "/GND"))
 (segment (start 111.625 56.5) (end 105.5 56.5) (width 1) (layer "B.Cu") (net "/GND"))
 (arc (start 114.625 63.5) (mid 113.56434 63.06066) (end 113.125 62) (width 1) (layer "B.Cu") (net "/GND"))
 (arc (start 113.125 58) (mid 112.68566 56.93934) (end 111.625 56.5) (width 1) (layer "B.Cu") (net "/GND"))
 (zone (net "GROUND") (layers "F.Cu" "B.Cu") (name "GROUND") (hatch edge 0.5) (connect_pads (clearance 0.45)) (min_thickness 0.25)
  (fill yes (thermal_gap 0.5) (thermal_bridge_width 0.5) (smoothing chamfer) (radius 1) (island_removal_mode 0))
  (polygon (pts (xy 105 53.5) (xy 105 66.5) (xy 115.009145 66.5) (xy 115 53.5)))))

